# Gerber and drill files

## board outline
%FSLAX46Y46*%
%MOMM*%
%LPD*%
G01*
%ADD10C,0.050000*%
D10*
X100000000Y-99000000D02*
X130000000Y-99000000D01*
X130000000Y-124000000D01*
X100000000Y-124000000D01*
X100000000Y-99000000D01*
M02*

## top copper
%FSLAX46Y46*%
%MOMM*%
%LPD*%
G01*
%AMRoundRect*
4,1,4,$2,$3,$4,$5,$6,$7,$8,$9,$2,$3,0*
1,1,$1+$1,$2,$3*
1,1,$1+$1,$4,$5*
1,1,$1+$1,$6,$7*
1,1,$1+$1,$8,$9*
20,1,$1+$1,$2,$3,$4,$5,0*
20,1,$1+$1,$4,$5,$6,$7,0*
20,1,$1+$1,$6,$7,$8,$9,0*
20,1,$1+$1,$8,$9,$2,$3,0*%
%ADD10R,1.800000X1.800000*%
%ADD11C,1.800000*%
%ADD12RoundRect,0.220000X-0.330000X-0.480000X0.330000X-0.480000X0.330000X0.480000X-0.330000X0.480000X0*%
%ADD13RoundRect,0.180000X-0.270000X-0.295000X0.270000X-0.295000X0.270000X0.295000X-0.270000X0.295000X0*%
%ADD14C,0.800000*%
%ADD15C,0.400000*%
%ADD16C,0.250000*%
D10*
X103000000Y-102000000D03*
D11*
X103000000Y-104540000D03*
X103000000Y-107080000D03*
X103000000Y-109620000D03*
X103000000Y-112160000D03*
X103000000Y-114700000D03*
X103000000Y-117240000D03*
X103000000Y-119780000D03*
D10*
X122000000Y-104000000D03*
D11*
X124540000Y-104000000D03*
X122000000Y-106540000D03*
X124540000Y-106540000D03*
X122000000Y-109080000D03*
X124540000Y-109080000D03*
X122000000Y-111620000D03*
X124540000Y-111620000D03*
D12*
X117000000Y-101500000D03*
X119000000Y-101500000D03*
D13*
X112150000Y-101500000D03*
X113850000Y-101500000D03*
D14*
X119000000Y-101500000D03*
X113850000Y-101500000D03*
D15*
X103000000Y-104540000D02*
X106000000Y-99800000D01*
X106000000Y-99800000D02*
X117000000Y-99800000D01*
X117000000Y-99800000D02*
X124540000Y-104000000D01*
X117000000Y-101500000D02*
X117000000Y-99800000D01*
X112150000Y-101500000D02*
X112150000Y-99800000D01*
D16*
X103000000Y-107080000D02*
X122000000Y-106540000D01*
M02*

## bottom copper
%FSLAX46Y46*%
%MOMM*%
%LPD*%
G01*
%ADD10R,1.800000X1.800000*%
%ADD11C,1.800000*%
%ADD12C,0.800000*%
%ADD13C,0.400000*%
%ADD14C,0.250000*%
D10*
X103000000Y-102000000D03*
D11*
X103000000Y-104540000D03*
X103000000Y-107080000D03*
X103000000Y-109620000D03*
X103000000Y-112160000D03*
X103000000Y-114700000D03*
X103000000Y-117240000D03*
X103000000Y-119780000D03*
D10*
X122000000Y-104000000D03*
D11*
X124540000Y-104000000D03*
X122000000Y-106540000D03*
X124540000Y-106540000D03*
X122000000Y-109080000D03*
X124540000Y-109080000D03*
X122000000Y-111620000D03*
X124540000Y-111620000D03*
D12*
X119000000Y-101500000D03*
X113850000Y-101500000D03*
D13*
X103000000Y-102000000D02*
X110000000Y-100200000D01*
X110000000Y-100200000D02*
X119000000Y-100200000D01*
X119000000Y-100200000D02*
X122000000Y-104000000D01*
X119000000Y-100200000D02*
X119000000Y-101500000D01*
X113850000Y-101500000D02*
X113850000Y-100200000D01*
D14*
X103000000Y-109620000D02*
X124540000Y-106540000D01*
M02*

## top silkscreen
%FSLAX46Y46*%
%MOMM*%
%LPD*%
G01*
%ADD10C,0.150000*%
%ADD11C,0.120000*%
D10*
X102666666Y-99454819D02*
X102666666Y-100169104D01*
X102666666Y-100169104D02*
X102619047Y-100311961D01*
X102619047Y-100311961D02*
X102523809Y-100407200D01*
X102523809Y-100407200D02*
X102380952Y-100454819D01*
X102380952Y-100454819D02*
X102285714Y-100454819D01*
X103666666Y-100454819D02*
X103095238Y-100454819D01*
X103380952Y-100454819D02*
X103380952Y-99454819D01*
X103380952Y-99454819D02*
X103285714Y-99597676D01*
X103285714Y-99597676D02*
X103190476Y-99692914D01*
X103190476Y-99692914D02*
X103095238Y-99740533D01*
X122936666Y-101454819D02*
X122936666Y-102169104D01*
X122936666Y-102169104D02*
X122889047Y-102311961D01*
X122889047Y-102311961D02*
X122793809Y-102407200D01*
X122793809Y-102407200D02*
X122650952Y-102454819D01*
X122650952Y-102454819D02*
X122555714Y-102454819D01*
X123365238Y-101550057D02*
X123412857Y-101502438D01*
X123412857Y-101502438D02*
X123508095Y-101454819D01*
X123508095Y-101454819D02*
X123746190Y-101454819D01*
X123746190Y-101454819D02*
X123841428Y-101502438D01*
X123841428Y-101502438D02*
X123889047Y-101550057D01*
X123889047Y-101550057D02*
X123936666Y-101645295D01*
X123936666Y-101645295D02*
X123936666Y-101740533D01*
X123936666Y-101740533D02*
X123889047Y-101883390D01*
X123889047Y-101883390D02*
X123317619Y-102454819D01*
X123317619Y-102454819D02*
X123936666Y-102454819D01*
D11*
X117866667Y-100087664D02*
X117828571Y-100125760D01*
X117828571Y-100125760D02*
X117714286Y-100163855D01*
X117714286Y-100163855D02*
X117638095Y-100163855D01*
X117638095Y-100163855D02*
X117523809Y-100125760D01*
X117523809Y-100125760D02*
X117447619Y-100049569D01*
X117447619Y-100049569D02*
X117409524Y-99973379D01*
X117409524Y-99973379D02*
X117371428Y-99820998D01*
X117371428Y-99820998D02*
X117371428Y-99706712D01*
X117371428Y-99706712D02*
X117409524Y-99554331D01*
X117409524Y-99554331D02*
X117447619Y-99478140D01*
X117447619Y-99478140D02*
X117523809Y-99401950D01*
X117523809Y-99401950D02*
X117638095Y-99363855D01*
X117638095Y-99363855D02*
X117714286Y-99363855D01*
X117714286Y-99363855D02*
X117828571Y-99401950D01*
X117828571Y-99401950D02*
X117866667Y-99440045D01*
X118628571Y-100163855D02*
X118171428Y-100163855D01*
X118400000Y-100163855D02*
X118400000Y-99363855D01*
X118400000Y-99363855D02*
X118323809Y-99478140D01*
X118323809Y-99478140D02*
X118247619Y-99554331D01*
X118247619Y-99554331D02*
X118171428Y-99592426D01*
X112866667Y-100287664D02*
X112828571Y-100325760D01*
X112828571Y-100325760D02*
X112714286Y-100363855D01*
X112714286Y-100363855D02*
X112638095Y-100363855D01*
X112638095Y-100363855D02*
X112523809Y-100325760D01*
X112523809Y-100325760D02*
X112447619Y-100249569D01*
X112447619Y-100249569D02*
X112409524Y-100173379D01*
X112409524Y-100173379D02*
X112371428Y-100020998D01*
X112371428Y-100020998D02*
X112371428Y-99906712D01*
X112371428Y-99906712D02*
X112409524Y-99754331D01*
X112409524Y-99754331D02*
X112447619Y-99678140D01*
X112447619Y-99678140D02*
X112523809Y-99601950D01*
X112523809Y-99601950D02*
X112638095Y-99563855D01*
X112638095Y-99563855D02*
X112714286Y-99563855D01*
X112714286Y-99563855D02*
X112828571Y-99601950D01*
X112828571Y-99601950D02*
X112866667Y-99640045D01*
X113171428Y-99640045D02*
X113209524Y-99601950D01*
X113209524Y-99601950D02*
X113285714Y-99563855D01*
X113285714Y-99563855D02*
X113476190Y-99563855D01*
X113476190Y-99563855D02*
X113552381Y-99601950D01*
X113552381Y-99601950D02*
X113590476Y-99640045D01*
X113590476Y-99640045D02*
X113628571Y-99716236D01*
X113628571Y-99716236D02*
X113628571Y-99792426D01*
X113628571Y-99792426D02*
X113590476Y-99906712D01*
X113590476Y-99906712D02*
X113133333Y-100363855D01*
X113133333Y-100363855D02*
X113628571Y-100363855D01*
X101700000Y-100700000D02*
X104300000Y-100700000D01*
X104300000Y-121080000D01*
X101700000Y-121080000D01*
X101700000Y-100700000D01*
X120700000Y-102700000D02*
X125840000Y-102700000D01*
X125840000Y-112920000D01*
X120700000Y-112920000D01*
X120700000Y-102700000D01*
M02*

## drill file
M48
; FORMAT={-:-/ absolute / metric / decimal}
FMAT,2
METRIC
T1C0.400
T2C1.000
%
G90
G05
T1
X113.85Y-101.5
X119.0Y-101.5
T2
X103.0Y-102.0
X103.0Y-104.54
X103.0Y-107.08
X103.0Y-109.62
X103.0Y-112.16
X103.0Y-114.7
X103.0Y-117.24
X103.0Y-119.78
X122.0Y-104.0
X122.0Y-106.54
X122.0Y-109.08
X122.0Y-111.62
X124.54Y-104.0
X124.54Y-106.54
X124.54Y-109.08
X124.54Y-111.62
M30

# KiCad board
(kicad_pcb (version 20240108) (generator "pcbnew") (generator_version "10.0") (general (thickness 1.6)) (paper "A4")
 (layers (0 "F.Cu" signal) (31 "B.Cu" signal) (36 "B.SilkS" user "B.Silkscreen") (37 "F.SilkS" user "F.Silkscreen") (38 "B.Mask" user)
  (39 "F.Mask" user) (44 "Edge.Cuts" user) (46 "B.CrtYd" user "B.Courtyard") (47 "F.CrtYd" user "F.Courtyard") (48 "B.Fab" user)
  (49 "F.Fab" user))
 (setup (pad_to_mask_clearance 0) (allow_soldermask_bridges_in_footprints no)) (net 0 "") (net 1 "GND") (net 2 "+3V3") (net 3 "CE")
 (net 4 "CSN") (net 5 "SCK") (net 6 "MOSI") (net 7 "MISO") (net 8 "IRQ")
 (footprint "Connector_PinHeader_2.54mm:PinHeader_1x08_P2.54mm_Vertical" (layer "F.Cu") (at 103 102)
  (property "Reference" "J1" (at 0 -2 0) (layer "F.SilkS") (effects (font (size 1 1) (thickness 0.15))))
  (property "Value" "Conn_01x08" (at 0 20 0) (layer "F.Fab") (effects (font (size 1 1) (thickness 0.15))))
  (fp_rect (start -1.3 -1.3) (end 1.3 19.08) (stroke (width 0.12) (type default)) (fill none) (layer "F.SilkS"))
  (pad "1" thru_hole rect (at 0 0) (size 1.8 1.8) (drill 1) (layers "*.Cu" "*.Mask") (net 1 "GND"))
  (pad "2" thru_hole circle (at 0 2.54) (size 1.8 1.8) (drill 1) (layers "*.Cu" "*.Mask") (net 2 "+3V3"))
  (pad "3" thru_hole circle (at 0 5.08) (size 1.8 1.8) (drill 1) (layers "*.Cu" "*.Mask") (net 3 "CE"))
  (pad "4" thru_hole circle (at 0 7.62) (size 1.8 1.8) (drill 1) (layers "*.Cu" "*.Mask") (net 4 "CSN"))
  (pad "5" thru_hole circle (at 0 10.16) (size 1.8 1.8) (drill 1) (layers "*.Cu" "*.Mask") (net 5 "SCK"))
  (pad "6" thru_hole circle (at 0 12.7) (size 1.8 1.8) (drill 1) (layers "*.Cu" "*.Mask") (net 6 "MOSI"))
  (pad "7" thru_hole circle (at 0 15.24) (size 1.8 1.8) (drill 1) (layers "*.Cu" "*.Mask") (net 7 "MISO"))
  (pad "8" thru_hole circle (at 0 17.78) (size 1.8 1.8) (drill 1) (layers "*.Cu" "*.Mask") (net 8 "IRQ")))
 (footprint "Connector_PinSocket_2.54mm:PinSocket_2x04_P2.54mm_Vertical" (layer "F.Cu") (at 122 104)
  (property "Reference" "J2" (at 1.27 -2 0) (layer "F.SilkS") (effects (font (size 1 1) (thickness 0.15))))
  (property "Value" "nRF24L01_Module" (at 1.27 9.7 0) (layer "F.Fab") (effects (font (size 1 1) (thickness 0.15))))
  (fp_rect (start -1.3 -1.3) (end 3.84 8.92) (stroke (width 0.12) (type default)) (fill none) (layer "F.SilkS"))
  (pad "1" thru_hole rect (at 0 0) (size 1.8 1.8) (drill 1) (layers "*.Cu" "*.Mask") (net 1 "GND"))
  (pad "2" thru_hole circle (at 2.54 0) (size 1.8 1.8) (drill 1) (layers "*.Cu" "*.Mask") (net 2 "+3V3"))
  (pad "3" thru_hole circle (at 0 2.54) (size 1.8 1.8) (drill 1) (layers "*.Cu" "*.Mask") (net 3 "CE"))
  (pad "4" thru_hole circle (at 2.54 2.54) (size 1.8 1.8) (drill 1) (layers "*.Cu" "*.Mask") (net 4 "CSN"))
  (pad "5" thru_hole circle (at 0 5.08) (size 1.8 1.8) (drill 1) (layers "*.Cu" "*.Mask") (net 5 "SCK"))
  (pad "6" thru_hole circle (at 2.54 5.08) (size 1.8 1.8) (drill 1) (layers "*.Cu" "*.Mask") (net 6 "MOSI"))
  (pad "7" thru_hole circle (at 0 7.62) (size 1.8 1.8) (drill 1) (layers "*.Cu" "*.Mask") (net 7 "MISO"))
  (pad "8" thru_hole circle (at 2.54 7.62) (size 1.8 1.8) (drill 1) (layers "*.Cu" "*.Mask") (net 8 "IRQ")))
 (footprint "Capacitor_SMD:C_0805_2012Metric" (layer "F.Cu") (at 118 101.5)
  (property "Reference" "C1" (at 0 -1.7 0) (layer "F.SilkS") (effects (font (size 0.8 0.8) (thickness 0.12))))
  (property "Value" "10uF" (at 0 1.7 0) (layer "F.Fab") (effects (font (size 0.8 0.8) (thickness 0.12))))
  (pad "1" smd roundrect (at -1 0) (size 1.1 1.4) (layers "F.Cu" "F.Paste" "F.Mask") (roundrect_rratio 0.2) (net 2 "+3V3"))
  (pad "2" smd roundrect (at 1 0) (size 1.1 1.4) (layers "F.Cu" "F.Paste" "F.Mask") (roundrect_rratio 0.2) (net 1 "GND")))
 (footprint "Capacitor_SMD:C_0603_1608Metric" (layer "F.Cu") (at 113 101.5)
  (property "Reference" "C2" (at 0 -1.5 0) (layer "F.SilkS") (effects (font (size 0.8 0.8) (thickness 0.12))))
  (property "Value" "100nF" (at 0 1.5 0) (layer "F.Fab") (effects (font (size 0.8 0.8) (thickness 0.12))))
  (pad "1" smd roundrect (at -0.85 0) (size 0.9 0.95) (layers "F.Cu" "F.Paste" "F.Mask") (roundrect_rratio 0.2) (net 2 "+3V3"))
  (pad "2" smd roundrect (at 0.85 0) (size 0.9 0.95) (layers "F.Cu" "F.Paste" "F.Mask") (roundrect_rratio 0.2) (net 1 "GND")))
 (gr_rect (start 100 99) (end 130 124) (stroke (width 0.05) (type default)) (fill none) (layer "Edge.Cuts"))
 (segment (start 103 102) (end 110 100.2) (width 0.4) (layer "B.Cu") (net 1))
 (segment (start 110 100.2) (end 119 100.2) (width 0.4) (layer "B.Cu") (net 1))
 (segment (start 119 100.2) (end 122 104) (width 0.4) (layer "B.Cu") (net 1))
 (segment (start 119 100.2) (end 119 101.5) (width 0.4) (layer "B.Cu") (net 1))
 (segment (start 113.85 101.5) (end 113.85 100.2) (width 0.4) (layer "B.Cu") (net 1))
 (segment (start 103 104.54) (end 106 99.8) (width 0.4) (layer "F.Cu") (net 2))
 (segment (start 106 99.8) (end 117 99.8) (width 0.4) (layer "F.Cu") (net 2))
 (segment (start 117 99.8) (end 124.54 104) (width 0.4) (layer "F.Cu") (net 2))
 (segment (start 117 101.5) (end 117 99.8) (width 0.4) (layer "F.Cu") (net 2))
 (segment (start 112.15 101.5) (end 112.15 99.8) (width 0.4) (layer "F.Cu") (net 2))
 (segment (start 103 107.08) (end 122 106.54) (width 0.25) (layer "F.Cu") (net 3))
 (segment (start 103 109.62) (end 124.54 106.54) (width 0.25) (layer "B.Cu") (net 4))
 (via (at 119 101.5) (size 0.8) (drill 0.4) (layers "F.Cu" "B.Cu") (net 1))
 (via (at 113.85 101.5) (size 0.8) (drill 0.4) (layers "F.Cu" "B.Cu") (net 1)))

